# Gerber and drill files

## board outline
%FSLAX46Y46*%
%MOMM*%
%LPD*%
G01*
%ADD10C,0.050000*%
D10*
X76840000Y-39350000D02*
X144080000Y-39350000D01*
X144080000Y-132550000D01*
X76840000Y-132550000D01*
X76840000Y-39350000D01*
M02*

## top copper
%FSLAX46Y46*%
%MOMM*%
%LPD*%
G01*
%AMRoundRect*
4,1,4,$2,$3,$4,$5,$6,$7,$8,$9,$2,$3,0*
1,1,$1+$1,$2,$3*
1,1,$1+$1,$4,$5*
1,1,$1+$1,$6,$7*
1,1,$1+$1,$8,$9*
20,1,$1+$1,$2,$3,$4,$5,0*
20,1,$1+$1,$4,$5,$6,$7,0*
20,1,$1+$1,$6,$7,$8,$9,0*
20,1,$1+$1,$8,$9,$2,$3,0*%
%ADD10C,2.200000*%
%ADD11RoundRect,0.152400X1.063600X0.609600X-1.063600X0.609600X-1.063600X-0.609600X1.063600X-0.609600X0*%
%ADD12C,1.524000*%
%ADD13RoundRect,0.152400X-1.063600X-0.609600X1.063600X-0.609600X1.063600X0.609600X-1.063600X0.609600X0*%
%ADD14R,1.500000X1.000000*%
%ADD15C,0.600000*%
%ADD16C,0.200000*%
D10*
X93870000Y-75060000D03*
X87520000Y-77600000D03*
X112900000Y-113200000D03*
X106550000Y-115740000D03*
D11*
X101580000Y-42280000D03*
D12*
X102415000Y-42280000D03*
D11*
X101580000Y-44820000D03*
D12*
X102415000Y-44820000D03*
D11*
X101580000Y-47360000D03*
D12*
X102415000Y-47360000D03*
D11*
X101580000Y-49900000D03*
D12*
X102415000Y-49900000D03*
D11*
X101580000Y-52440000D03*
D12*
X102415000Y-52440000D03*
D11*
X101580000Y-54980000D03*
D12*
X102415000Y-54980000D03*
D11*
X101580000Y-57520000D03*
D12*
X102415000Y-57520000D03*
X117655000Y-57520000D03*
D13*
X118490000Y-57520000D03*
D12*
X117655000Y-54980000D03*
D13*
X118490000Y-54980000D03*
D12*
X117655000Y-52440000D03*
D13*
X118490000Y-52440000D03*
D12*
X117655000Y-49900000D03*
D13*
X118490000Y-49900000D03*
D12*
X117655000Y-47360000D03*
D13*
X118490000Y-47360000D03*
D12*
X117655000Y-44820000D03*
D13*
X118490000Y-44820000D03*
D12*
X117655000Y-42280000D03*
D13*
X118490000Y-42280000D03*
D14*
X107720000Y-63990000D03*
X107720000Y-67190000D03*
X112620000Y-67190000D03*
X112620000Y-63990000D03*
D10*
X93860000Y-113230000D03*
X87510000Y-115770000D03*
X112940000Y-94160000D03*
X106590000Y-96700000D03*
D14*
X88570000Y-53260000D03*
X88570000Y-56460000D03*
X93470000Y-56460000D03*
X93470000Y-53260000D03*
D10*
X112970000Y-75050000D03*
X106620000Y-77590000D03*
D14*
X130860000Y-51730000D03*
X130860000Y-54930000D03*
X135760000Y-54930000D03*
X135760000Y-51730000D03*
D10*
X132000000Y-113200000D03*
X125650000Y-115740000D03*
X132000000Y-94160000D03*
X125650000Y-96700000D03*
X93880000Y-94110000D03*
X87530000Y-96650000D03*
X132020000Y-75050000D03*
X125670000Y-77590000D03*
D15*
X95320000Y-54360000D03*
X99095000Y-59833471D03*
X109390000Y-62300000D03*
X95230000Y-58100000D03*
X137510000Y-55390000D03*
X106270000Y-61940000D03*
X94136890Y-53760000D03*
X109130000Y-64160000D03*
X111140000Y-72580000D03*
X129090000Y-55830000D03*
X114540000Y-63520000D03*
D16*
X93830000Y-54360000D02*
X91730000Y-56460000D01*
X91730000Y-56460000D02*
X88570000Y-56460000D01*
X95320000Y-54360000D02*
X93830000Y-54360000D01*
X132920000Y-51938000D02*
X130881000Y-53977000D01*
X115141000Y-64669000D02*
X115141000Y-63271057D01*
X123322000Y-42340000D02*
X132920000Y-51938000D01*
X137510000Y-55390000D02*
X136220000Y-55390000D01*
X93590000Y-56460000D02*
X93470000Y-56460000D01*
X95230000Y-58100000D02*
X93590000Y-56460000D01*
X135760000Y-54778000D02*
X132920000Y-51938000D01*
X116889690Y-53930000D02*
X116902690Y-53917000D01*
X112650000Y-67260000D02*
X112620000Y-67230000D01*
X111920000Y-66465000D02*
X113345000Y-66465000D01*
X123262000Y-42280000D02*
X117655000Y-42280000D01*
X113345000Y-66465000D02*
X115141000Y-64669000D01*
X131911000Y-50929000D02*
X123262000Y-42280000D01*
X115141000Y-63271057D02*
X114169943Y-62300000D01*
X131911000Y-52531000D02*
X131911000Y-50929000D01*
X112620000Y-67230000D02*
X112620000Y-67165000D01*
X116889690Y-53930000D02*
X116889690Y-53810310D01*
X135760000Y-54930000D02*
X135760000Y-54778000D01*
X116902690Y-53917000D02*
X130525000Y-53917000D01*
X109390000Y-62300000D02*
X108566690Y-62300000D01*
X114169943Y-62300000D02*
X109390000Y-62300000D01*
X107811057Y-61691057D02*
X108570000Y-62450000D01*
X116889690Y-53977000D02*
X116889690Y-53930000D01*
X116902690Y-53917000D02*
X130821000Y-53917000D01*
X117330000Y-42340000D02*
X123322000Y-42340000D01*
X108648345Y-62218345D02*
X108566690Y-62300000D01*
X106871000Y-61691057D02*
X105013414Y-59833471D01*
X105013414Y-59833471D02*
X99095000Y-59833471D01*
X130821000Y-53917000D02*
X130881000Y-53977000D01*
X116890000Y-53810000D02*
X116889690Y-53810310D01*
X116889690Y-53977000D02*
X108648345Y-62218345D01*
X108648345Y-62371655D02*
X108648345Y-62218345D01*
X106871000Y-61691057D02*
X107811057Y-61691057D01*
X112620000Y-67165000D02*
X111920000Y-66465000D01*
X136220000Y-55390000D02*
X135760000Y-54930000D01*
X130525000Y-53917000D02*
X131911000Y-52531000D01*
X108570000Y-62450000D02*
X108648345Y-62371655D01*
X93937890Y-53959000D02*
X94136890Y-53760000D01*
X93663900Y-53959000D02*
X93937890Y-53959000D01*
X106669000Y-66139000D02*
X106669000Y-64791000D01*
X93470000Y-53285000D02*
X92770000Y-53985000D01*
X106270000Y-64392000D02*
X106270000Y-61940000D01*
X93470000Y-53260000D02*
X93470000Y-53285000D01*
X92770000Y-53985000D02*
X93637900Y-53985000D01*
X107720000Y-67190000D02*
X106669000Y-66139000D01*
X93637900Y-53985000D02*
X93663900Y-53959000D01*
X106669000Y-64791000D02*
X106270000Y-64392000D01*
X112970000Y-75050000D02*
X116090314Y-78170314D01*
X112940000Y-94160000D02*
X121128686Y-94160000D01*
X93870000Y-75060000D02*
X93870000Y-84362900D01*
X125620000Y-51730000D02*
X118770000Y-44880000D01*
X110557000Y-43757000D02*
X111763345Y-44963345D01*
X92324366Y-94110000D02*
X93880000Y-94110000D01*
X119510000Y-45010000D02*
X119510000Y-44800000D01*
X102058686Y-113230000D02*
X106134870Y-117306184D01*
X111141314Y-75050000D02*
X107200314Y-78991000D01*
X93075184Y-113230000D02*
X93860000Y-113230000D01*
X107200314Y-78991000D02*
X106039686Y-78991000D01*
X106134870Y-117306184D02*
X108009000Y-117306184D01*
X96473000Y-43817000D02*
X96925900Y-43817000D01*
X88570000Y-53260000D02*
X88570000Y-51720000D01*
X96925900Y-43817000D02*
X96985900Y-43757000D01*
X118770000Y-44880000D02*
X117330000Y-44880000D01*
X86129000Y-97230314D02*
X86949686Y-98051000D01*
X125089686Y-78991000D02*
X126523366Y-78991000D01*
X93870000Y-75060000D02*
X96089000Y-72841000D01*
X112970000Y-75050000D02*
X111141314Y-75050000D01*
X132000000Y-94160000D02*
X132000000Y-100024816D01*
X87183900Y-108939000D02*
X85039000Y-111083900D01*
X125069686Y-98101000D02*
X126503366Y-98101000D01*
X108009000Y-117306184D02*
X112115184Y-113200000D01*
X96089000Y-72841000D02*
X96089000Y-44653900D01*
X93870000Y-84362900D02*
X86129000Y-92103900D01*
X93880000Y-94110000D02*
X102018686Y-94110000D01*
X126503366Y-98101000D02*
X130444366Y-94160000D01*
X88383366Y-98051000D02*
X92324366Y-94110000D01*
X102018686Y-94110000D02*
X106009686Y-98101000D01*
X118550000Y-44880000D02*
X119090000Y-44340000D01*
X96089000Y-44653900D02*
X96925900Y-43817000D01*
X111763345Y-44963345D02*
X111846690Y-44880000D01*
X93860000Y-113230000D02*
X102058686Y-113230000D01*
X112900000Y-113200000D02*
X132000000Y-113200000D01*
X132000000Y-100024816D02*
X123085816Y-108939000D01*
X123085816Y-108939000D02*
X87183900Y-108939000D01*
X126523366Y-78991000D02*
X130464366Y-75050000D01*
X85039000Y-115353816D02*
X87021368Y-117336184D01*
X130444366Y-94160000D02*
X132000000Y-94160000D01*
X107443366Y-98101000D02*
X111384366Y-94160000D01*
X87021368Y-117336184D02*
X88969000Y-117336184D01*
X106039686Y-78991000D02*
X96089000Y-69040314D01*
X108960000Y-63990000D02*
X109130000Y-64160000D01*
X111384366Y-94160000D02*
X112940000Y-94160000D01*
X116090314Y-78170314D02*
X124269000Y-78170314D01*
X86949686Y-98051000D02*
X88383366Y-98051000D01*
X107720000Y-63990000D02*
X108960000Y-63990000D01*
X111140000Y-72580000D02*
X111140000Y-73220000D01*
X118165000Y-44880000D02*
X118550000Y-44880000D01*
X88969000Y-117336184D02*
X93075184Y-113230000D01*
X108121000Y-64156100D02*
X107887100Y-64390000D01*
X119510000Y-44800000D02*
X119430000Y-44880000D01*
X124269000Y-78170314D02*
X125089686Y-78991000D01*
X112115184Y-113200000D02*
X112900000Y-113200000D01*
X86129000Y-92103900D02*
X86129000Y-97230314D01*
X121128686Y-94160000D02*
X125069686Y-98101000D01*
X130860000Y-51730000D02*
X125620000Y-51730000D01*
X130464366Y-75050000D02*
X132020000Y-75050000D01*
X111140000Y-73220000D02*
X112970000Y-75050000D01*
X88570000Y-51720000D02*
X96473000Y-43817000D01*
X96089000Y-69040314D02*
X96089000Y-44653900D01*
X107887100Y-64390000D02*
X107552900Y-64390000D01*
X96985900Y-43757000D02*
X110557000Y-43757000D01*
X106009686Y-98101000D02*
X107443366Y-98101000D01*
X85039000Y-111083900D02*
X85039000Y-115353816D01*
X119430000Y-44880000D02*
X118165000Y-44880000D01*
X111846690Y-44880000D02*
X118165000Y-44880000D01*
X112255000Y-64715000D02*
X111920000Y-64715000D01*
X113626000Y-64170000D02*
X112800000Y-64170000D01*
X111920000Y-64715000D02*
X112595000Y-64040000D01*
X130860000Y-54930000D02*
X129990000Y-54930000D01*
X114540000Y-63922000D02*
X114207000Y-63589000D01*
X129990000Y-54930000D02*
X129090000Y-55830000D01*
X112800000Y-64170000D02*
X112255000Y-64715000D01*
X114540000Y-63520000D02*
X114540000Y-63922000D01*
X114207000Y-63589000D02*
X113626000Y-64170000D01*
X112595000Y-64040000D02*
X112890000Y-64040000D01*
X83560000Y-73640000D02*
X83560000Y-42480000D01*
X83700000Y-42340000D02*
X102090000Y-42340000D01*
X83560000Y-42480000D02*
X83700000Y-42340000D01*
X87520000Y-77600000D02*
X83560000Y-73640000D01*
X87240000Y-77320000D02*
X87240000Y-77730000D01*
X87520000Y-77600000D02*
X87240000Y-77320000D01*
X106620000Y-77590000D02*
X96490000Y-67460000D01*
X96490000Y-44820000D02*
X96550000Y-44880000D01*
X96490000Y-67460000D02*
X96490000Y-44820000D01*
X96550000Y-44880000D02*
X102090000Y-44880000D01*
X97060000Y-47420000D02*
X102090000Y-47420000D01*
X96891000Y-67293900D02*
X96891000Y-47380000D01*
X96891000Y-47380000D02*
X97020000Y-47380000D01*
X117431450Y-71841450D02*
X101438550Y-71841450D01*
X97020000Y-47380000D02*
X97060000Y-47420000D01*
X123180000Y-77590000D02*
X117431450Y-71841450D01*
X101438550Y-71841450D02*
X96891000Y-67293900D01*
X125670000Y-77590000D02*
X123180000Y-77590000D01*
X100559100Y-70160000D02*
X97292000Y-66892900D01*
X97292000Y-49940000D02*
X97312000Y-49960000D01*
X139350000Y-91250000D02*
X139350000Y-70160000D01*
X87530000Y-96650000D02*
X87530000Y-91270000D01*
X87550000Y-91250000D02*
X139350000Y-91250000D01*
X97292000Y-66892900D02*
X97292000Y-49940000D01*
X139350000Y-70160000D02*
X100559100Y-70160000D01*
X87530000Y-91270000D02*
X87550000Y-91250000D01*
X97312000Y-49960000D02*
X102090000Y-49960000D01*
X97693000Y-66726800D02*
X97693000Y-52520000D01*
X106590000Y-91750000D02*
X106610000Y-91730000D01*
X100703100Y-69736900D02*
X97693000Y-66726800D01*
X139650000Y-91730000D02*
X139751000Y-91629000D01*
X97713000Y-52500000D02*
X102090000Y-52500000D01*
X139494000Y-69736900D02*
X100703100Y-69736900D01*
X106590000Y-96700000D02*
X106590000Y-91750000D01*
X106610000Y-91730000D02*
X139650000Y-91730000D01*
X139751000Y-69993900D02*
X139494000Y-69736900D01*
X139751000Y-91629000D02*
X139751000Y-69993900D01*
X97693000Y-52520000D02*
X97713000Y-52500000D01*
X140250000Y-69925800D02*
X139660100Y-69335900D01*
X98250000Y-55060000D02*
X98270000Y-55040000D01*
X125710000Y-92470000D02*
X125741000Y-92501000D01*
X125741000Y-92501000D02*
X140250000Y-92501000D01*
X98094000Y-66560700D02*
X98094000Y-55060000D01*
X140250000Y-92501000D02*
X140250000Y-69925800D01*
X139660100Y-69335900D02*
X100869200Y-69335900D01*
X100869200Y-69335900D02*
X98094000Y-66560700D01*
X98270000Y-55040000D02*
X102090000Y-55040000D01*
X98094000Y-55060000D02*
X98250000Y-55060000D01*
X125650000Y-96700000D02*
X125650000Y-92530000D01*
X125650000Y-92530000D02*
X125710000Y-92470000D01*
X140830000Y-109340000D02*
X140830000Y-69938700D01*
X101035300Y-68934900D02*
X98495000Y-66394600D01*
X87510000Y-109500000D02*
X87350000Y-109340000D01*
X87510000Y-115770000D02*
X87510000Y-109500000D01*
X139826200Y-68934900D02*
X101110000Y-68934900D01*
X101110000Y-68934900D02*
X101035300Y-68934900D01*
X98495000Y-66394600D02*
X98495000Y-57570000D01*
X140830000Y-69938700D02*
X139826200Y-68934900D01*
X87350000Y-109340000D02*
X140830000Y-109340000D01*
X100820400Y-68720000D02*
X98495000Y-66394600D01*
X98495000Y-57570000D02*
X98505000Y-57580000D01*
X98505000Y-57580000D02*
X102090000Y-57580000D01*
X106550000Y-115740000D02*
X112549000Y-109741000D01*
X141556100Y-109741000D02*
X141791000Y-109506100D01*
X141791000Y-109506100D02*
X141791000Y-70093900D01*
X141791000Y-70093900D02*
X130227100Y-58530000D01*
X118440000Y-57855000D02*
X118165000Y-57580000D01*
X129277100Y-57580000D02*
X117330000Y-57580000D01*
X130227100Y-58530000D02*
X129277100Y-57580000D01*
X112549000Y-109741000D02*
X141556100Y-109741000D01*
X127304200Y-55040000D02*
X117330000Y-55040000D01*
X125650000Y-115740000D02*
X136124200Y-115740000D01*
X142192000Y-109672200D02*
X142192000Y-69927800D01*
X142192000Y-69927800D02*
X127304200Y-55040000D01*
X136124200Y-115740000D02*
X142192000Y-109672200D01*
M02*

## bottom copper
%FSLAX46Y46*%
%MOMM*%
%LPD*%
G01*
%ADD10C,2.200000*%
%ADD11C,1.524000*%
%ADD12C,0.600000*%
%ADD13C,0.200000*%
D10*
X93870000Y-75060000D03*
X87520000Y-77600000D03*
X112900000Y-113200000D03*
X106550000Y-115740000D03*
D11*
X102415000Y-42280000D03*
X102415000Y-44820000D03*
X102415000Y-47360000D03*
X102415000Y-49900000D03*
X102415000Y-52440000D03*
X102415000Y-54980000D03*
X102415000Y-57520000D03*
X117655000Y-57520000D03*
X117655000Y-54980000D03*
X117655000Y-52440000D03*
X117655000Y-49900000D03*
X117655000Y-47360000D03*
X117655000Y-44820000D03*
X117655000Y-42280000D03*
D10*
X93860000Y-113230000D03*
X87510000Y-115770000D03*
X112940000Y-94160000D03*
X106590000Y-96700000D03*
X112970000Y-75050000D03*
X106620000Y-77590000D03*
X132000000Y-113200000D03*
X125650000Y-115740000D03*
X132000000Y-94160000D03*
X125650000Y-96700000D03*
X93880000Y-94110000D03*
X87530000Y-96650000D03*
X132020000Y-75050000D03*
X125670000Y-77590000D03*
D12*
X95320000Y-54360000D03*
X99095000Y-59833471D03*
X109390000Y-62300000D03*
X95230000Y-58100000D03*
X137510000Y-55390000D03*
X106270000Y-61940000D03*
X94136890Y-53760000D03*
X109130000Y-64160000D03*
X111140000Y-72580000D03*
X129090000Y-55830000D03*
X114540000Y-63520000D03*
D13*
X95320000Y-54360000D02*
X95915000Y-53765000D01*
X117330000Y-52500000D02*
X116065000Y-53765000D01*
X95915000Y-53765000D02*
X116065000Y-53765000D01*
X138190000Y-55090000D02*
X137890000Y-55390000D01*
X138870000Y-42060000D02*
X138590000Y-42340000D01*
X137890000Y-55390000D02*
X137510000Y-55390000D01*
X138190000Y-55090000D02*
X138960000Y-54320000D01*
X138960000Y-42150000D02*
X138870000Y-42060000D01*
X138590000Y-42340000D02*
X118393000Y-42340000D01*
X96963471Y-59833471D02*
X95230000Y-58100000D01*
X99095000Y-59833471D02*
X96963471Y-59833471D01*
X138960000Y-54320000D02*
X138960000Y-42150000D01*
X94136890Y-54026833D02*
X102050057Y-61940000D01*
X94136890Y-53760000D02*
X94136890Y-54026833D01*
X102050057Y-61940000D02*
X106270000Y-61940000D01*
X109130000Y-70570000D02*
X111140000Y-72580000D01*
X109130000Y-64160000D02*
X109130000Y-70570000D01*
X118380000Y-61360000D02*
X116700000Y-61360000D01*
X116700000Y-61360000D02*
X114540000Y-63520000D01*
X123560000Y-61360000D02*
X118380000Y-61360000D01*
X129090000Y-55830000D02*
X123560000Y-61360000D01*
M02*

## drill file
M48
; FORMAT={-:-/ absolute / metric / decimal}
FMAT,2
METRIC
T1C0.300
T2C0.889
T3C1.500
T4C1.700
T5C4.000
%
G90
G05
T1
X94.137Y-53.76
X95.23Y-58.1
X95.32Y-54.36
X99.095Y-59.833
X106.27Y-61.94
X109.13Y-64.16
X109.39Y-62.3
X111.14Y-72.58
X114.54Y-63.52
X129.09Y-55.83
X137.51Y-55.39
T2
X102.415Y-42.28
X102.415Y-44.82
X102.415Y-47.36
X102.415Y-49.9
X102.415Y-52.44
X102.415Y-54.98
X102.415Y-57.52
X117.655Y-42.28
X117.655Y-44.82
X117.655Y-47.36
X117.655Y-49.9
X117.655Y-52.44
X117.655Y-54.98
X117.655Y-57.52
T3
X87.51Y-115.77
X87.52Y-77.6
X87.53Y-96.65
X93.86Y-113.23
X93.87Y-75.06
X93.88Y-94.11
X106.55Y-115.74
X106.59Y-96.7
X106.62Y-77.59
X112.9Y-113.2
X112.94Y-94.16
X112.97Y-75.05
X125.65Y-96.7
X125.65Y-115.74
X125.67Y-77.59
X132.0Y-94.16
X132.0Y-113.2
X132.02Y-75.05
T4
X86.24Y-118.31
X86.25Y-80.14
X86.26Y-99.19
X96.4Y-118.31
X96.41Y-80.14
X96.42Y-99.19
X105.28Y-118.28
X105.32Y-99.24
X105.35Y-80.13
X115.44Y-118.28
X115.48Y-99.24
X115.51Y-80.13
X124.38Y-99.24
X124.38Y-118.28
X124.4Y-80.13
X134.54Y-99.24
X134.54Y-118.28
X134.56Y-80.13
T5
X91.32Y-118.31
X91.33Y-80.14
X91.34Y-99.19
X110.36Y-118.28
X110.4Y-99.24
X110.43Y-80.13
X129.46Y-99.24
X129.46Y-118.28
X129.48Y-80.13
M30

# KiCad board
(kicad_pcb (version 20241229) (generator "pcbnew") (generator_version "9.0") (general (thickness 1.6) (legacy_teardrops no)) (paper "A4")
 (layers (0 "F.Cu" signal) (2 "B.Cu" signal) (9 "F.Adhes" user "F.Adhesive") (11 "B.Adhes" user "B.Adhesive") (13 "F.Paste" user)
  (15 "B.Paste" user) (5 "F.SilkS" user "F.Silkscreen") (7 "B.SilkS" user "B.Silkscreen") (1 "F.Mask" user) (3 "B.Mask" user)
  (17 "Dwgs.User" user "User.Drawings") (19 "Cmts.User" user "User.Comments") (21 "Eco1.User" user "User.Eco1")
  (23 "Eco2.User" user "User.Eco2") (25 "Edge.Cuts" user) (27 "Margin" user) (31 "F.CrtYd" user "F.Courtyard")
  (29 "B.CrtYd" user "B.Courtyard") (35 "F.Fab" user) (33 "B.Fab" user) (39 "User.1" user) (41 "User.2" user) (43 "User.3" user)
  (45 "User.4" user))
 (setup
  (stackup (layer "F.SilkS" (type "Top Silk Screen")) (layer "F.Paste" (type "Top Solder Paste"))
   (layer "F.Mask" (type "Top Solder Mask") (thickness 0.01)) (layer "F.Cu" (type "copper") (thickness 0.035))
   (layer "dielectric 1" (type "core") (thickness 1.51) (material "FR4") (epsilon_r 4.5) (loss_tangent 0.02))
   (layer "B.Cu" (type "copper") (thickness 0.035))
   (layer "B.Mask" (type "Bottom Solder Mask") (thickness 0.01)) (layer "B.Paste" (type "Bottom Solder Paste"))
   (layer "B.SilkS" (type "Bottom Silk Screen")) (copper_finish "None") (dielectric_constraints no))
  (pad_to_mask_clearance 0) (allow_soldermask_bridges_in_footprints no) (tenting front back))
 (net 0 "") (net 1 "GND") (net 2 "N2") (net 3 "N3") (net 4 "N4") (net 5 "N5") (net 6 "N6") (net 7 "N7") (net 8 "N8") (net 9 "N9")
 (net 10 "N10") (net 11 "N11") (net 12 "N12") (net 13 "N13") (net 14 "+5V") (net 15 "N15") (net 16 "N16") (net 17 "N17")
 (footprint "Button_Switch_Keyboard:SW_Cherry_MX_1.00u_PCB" (layer "F.Cu") (at 93.87 75.06)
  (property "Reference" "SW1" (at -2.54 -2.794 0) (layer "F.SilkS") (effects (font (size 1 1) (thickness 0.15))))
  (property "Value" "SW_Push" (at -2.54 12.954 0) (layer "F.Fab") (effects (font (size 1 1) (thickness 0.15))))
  (pad "" np_thru_hole circle (at -7.62 5.08) (size 1.7 1.7) (drill 1.7) (layers "*.Cu" "*.Mask"))
  (pad "" np_thru_hole circle (at -2.54 5.08) (size 4 4) (drill 4) (layers "*.Cu" "*.Mask"))
  (pad "" np_thru_hole circle (at 2.54 5.08) (size 1.7 1.7) (drill 1.7) (layers "*.Cu" "*.Mask"))
  (pad "1" thru_hole circle (at 0 0) (size 2.2 2.2) (drill 1.5) (layers "*.Cu" "*.Mask") (remove_unused_layers no) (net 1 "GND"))
  (pad "2" thru_hole circle (at -6.35 2.54) (size 2.2 2.2) (drill 1.5) (layers "*.Cu" "*.Mask") (remove_unused_layers no) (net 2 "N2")))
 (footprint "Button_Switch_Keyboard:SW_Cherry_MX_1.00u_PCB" (layer "F.Cu") (at 112.9 113.2)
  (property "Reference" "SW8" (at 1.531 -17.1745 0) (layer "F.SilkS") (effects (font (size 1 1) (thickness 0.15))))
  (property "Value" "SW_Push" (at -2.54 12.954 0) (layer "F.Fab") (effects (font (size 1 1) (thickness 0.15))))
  (pad "" np_thru_hole circle (at -7.62 5.08) (size 1.7 1.7) (drill 1.7) (layers "*.Cu" "*.Mask"))
  (pad "" np_thru_hole circle (at -2.54 5.08) (size 4 4) (drill 4) (layers "*.Cu" "*.Mask"))
  (pad "" np_thru_hole circle (at 2.54 5.08) (size 1.7 1.7) (drill 1.7) (layers "*.Cu" "*.Mask"))
  (pad "1" thru_hole circle (at 0 0) (size 2.2 2.2) (drill 1.5) (layers "*.Cu" "*.Mask") (remove_unused_layers no) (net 1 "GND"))
  (pad "2" thru_hole circle (at -6.35 2.54) (size 2.2 2.2) (drill 1.5) (layers "*.Cu" "*.Mask") (remove_unused_layers no) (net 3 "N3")))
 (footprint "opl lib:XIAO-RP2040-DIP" (layer "F.Cu") (at 110.035 49.9)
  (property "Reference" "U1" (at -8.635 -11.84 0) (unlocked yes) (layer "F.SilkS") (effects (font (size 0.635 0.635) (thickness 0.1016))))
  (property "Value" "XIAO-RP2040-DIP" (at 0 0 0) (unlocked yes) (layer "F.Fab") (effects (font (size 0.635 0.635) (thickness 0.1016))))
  (pad "1" smd roundrect (at -8.455 -7.62 180) (size 2.432 1.524) (layers "F.Cu" "F.Mask") (roundrect_rratio 0.1) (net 2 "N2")
   (thermal_bridge_angle 45))
  (pad "1" thru_hole circle (at -7.62 -7.62 180) (size 1.524 1.524) (drill 0.889) (layers "*.Cu" "*.Mask") (remove_unused_layers no)
   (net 2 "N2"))
  (pad "2" smd roundrect (at -8.455 -5.08 180) (size 2.432 1.524) (layers "F.Cu" "F.Mask") (roundrect_rratio 0.1) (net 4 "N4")
   (thermal_bridge_angle 45))
  (pad "2" thru_hole circle (at -7.62 -5.08 180) (size 1.524 1.524) (drill 0.889) (layers "*.Cu" "*.Mask") (remove_unused_layers no)
   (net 4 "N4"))
  (pad "3" smd roundrect (at -8.455 -2.54 180) (size 2.432 1.524) (layers "F.Cu" "F.Mask") (roundrect_rratio 0.1) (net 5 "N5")
   (thermal_bridge_angle 45))
  (pad "3" thru_hole circle (at -7.62 -2.54 180) (size 1.524 1.524) (drill 0.889) (layers "*.Cu" "*.Mask") (remove_unused_layers no)
   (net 5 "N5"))
  (pad "4" smd roundrect (at -8.455 0 180) (size 2.432 1.524) (layers "F.Cu" "F.Mask") (roundrect_rratio 0.1) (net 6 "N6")
   (thermal_bridge_angle 45))
  (pad "4" thru_hole circle (at -7.62 0 180) (size 1.524 1.524) (drill 0.889) (layers "*.Cu" "*.Mask") (remove_unused_layers no)
   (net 6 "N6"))
  (pad "5" smd roundrect (at -8.455 2.54 180) (size 2.432 1.524) (layers "F.Cu" "F.Mask") (roundrect_rratio 0.1) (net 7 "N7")
   (thermal_bridge_angle 45))
  (pad "5" thru_hole circle (at -7.62 2.54 180) (size 1.524 1.524) (drill 0.889) (layers "*.Cu" "*.Mask") (remove_unused_layers no)
   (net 7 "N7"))
  (pad "6" smd roundrect (at -8.455 5.08 180) (size 2.432 1.524) (layers "F.Cu" "F.Mask") (roundrect_rratio 0.1) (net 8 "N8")
   (thermal_bridge_angle 45))
  (pad "6" thru_hole circle (at -7.62 5.08 180) (size 1.524 1.524) (drill 0.889) (layers "*.Cu" "*.Mask") (remove_unused_layers no)
   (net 8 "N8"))
  (pad "7" smd roundrect (at -8.455 7.62 180) (size 2.432 1.524) (layers "F.Cu" "F.Mask") (roundrect_rratio 0.1) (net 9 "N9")
   (thermal_bridge_angle 45))
  (pad "7" thru_hole circle (at -7.62 7.62 180) (size 1.524 1.524) (drill 0.889) (layers "*.Cu" "*.Mask") (remove_unused_layers no)
   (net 9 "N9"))
  (pad "8" thru_hole circle (at 7.62 7.62) (size 1.524 1.524) (drill 0.889) (layers "*.Cu" "*.Mask") (remove_unused_layers no) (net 3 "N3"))
  (pad "8" smd roundrect (at 8.455 7.62) (size 2.432 1.524) (layers "F.Cu" "F.Mask") (roundrect_rratio 0.1) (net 3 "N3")
   (thermal_bridge_angle 45))
  (pad "9" thru_hole circle (at 7.62 5.08) (size 1.524 1.524) (drill 0.889) (layers "*.Cu" "*.Mask") (remove_unused_layers no)
   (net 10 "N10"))
  (pad "9" smd roundrect (at 8.455 5.08) (size 2.432 1.524) (layers "F.Cu" "F.Mask") (roundrect_rratio 0.1) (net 10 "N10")
   (thermal_bridge_angle 45))
  (pad "10" thru_hole circle (at 7.62 2.54) (size 1.524 1.524) (drill 0.889) (layers "*.Cu" "*.Mask") (remove_unused_layers no)
   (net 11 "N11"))
  (pad "10" smd roundrect (at 8.455 2.54) (size 2.432 1.524) (layers "F.Cu" "F.Mask") (roundrect_rratio 0.1) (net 11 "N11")
   (thermal_bridge_angle 45))
  (pad "11" thru_hole circle (at 7.62 0) (size 1.524 1.524) (drill 0.889) (layers "*.Cu" "*.Mask") (remove_unused_layers no) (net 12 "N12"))
  (pad "11" smd roundrect (at 8.455 0) (size 2.432 1.524) (layers "F.Cu" "F.Mask") (roundrect_rratio 0.1) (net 12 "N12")
   (thermal_bridge_angle 45))
  (pad "12" thru_hole circle (at 7.62 -2.54) (size 1.524 1.524) (drill 0.889) (layers "*.Cu" "*.Mask") (remove_unused_layers no)
   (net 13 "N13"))
  (pad "12" smd roundrect (at 8.455 -2.54) (size 2.432 1.524) (layers "F.Cu" "F.Mask") (roundrect_rratio 0.1) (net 13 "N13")
   (thermal_bridge_angle 45))
  (pad "13" thru_hole circle (at 7.62 -5.08) (size 1.524 1.524) (drill 0.889) (layers "*.Cu" "*.Mask") (remove_unused_layers no)
   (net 1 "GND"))
  (pad "13" smd roundrect (at 8.455 -5.08) (size 2.432 1.524) (layers "F.Cu" "F.Mask") (roundrect_rratio 0.1) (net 1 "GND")
   (thermal_bridge_angle 45))
  (pad "14" thru_hole circle (at 7.62 -7.62) (size 1.524 1.524) (drill 0.889) (layers "*.Cu" "*.Mask") (remove_unused_layers no)
   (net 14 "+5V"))
  (pad "14" smd roundrect (at 8.455 -7.62) (size 2.432 1.524) (layers "F.Cu" "F.Mask") (roundrect_rratio 0.1) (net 14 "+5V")
   (thermal_bridge_angle 45)))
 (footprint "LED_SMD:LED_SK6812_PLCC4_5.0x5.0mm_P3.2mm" (layer "F.Cu") (at 110.17 65.59)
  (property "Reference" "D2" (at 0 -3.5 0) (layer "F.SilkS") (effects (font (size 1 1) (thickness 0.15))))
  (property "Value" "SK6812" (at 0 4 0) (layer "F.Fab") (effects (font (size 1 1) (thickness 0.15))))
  (pad "1" smd rect (at -2.45 -1.6 180) (size 1.5 1) (layers "F.Cu" "F.Mask" "F.Paste") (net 1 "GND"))
  (pad "2" smd rect (at -2.45 1.6 180) (size 1.5 1) (layers "F.Cu" "F.Mask" "F.Paste") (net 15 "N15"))
  (pad "3" smd rect (at 2.45 1.6 180) (size 1.5 1) (layers "F.Cu" "F.Mask" "F.Paste") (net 14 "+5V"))
  (pad "4" smd rect (at 2.45 -1.6 180) (size 1.5 1) (layers "F.Cu" "F.Mask" "F.Paste") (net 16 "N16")))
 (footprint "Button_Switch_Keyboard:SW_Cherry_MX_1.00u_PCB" (layer "F.Cu") (at 93.86 113.23)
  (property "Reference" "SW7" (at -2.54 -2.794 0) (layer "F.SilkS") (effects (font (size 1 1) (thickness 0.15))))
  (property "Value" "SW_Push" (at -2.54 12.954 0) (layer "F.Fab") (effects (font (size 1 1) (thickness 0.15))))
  (pad "" np_thru_hole circle (at -7.62 5.08) (size 1.7 1.7) (drill 1.7) (layers "*.Cu" "*.Mask"))
  (pad "" np_thru_hole circle (at -2.54 5.08) (size 4 4) (drill 4) (layers "*.Cu" "*.Mask"))
  (pad "" np_thru_hole circle (at 2.54 5.08) (size 1.7 1.7) (drill 1.7) (layers "*.Cu" "*.Mask"))
  (pad "1" thru_hole circle (at 0 0) (size 2.2 2.2) (drill 1.5) (layers "*.Cu" "*.Mask") (remove_unused_layers no) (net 1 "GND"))
  (pad "2" thru_hole circle (at -6.35 2.54) (size 2.2 2.2) (drill 1.5) (layers "*.Cu" "*.Mask") (remove_unused_layers no) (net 9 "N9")))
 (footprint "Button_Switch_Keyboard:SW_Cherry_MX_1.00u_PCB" (layer "F.Cu") (at 112.94 94.16)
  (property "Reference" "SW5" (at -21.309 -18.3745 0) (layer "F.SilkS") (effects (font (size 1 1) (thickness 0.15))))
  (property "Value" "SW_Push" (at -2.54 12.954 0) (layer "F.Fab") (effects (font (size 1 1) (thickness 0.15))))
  (pad "" np_thru_hole circle (at -7.62 5.08) (size 1.7 1.7) (drill 1.7) (layers "*.Cu" "*.Mask"))
  (pad "" np_thru_hole circle (at -2.54 5.08) (size 4 4) (drill 4) (layers "*.Cu" "*.Mask"))
  (pad "" np_thru_hole circle (at 2.54 5.08) (size 1.7 1.7) (drill 1.7) (layers "*.Cu" "*.Mask"))
  (pad "1" thru_hole circle (at 0 0) (size 2.2 2.2) (drill 1.5) (layers "*.Cu" "*.Mask") (remove_unused_layers no) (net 1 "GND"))
  (pad "2" thru_hole circle (at -6.35 2.54) (size 2.2 2.2) (drill 1.5) (layers "*.Cu" "*.Mask") (remove_unused_layers no) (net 7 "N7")))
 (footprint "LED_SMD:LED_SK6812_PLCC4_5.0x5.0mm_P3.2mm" (layer "F.Cu") (at 91.02 54.86)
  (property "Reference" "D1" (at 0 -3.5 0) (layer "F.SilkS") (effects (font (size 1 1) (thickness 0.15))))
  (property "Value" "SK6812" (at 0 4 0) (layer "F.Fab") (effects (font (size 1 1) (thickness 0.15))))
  (pad "1" smd rect (at -2.45 -1.6 180) (size 1.5 1) (layers "F.Cu" "F.Mask" "F.Paste") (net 1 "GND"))
  (pad "2" smd rect (at -2.45 1.6 180) (size 1.5 1) (layers "F.Cu" "F.Mask" "F.Paste") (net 11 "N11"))
  (pad "3" smd rect (at 2.45 1.6 180) (size 1.5 1) (layers "F.Cu" "F.Mask" "F.Paste") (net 14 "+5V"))
  (pad "4" smd rect (at 2.45 -1.6 180) (size 1.5 1) (layers "F.Cu" "F.Mask" "F.Paste") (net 15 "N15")))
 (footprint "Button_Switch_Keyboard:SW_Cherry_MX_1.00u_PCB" (layer "F.Cu") (at 112.97 75.05)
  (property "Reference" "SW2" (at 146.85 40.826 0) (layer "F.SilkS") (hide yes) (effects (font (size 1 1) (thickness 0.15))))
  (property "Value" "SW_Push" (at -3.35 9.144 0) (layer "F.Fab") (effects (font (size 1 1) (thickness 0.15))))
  (pad "" np_thru_hole circle (at -7.62 5.08) (size 1.7 1.7) (drill 1.7) (layers "*.Cu" "*.Mask"))
  (pad "" np_thru_hole circle (at -2.54 5.08) (size 4 4) (drill 4) (layers "*.Cu" "*.Mask"))
  (pad "" np_thru_hole circle (at 2.54 5.08) (size 1.7 1.7) (drill 1.7) (layers "*.Cu" "*.Mask"))
  (pad "1" thru_hole circle (at 0 0) (size 2.2 2.2) (drill 1.5) (layers "*.Cu" "*.Mask") (remove_unused_layers no) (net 1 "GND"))
  (pad "2" thru_hole circle (at -6.35 2.54) (size 2.2 2.2) (drill 1.5) (layers "*.Cu" "*.Mask") (remove_unused_layers no) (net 4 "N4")))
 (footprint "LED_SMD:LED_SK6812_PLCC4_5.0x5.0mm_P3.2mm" (layer "F.Cu") (at 133.31 53.33)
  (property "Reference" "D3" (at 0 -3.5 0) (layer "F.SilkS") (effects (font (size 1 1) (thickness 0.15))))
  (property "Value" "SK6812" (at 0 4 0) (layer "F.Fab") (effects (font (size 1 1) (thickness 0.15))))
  (pad "1" smd rect (at -2.45 -1.6 180) (size 1.5 1) (layers "F.Cu" "F.Mask" "F.Paste") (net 1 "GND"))
  (pad "2" smd rect (at -2.45 1.6 180) (size 1.5 1) (layers "F.Cu" "F.Mask" "F.Paste") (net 16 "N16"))
  (pad "3" smd rect (at 2.45 1.6 180) (size 1.5 1) (layers "F.Cu" "F.Mask" "F.Paste") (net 14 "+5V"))
  (pad "4" smd rect (at 2.45 -1.6 180) (size 1.5 1) (layers "F.Cu" "F.Mask" "F.Paste") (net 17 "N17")))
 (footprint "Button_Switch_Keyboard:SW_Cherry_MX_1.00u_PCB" (layer "F.Cu") (at 132 113.2)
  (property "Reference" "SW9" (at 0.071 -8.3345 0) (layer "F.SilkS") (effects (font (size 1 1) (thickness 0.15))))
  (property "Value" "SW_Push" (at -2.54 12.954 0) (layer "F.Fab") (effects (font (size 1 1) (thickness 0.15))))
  (pad "" np_thru_hole circle (at -7.62 5.08) (size 1.7 1.7) (drill 1.7) (layers "*.Cu" "*.Mask"))
  (pad "" np_thru_hole circle (at -2.54 5.08) (size 4 4) (drill 4) (layers "*.Cu" "*.Mask"))
  (pad "" np_thru_hole circle (at 2.54 5.08) (size 1.7 1.7) (drill 1.7) (layers "*.Cu" "*.Mask"))
  (pad "1" thru_hole circle (at 0 0) (size 2.2 2.2) (drill 1.5) (layers "*.Cu" "*.Mask") (remove_unused_layers no) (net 1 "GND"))
  (pad "2" thru_hole circle (at -6.35 2.54) (size 2.2 2.2) (drill 1.5) (layers "*.Cu" "*.Mask") (remove_unused_layers no) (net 10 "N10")))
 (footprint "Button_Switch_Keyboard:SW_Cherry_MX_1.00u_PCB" (layer "F.Cu") (at 132 94.16)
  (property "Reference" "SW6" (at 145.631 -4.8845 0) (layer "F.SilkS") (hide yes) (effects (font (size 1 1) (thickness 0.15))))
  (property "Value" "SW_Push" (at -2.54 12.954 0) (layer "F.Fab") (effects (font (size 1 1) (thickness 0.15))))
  (pad "" np_thru_hole circle (at -7.62 5.08) (size 1.7 1.7) (drill 1.7) (layers "*.Cu" "*.Mask"))
  (pad "" np_thru_hole circle (at -2.54 5.08) (size 4 4) (drill 4) (layers "*.Cu" "*.Mask"))
  (pad "" np_thru_hole circle (at 2.54 5.08) (size 1.7 1.7) (drill 1.7) (layers "*.Cu" "*.Mask"))
  (pad "1" thru_hole circle (at 0 0) (size 2.2 2.2) (drill 1.5) (layers "*.Cu" "*.Mask") (remove_unused_layers no) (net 1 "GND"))
  (pad "2" thru_hole circle (at -6.35 2.54) (size 2.2 2.2) (drill 1.5) (layers "*.Cu" "*.Mask") (remove_unused_layers no) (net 8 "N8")))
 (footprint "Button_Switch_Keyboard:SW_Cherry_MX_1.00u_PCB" (layer "F.Cu") (at 93.88 94.11)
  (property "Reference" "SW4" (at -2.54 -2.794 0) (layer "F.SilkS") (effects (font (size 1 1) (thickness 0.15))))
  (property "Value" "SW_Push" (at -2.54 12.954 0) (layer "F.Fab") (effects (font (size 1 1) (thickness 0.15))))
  (pad "" np_thru_hole circle (at -7.62 5.08) (size 1.7 1.7) (drill 1.7) (layers "*.Cu" "*.Mask"))
  (pad "" np_thru_hole circle (at -2.54 5.08) (size 4 4) (drill 4) (layers "*.Cu" "*.Mask"))
  (pad "" np_thru_hole circle (at 2.54 5.08) (size 1.7 1.7) (drill 1.7) (layers "*.Cu" "*.Mask"))
  (pad "1" thru_hole circle (at 0 0) (size 2.2 2.2) (drill 1.5) (layers "*.Cu" "*.Mask") (remove_unused_layers no) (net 1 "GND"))
  (pad "2" thru_hole circle (at -6.35 2.54) (size 2.2 2.2) (drill 1.5) (layers "*.Cu" "*.Mask") (remove_unused_layers no) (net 6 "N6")))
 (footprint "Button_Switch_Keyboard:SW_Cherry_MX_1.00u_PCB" (layer "F.Cu") (at 132.02 75.05)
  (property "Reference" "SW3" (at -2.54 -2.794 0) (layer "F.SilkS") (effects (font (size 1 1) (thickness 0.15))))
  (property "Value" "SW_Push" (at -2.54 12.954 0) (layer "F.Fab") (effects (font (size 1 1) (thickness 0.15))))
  (pad "" np_thru_hole circle (at -7.62 5.08) (size 1.7 1.7) (drill 1.7) (layers "*.Cu" "*.Mask"))
  (pad "" np_thru_hole circle (at -2.54 5.08) (size 4 4) (drill 4) (layers "*.Cu" "*.Mask"))
  (pad "" np_thru_hole circle (at 2.54 5.08) (size 1.7 1.7) (drill 1.7) (layers "*.Cu" "*.Mask"))
  (pad "1" thru_hole circle (at 0 0) (size 2.2 2.2) (drill 1.5) (layers "*.Cu" "*.Mask") (remove_unused_layers no) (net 1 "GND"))
  (pad "2" thru_hole circle (at -6.35 2.54) (size 2.2 2.2) (drill 1.5) (layers "*.Cu" "*.Mask") (remove_unused_layers no) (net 5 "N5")))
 (gr_rect (start 76.84 39.35) (end 144.08 132.55) (stroke (width 0.05) (type default)) (fill no) (layer "Edge.Cuts"))
 (segment (start 93.83 54.36) (end 91.73 56.46) (width 0.2) (layer "F.Cu") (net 11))
 (segment (start 91.73 56.46) (end 88.57 56.46) (width 0.2) (layer "F.Cu") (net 11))
 (segment (start 95.32 54.36) (end 93.83 54.36) (width 0.2) (layer "F.Cu") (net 11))
 (via (at 95.32 54.36) (size 0.6) (drill 0.3) (layers "F.Cu" "B.Cu") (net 11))
 (segment (start 95.32 54.36) (end 95.915 53.765) (width 0.2) (layer "B.Cu") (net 11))
 (segment (start 117.33 52.5) (end 116.065 53.765) (width 0.2) (layer "B.Cu") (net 11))
 (segment (start 95.915 53.765) (end 116.065 53.765) (width 0.2) (layer "B.Cu") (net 11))
 (segment (start 132.92 51.938) (end 130.881 53.977) (width 0.2) (layer "F.Cu") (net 14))
 (segment (start 115.141 64.669) (end 115.141 63.271057) (width 0.2) (layer "F.Cu") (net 14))
 (segment (start 123.322 42.34) (end 132.92 51.938) (width 0.2) (layer "F.Cu") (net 14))
 (segment (start 137.51 55.39) (end 136.22 55.39) (width 0.2) (layer "F.Cu") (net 14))
 (segment (start 93.59 56.46) (end 93.47 56.46) (width 0.2) (layer "F.Cu") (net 14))
 (segment (start 95.23 58.1) (end 93.59 56.46) (width 0.2) (layer "F.Cu") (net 14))
 (segment (start 135.76 54.778) (end 132.92 51.938) (width 0.2) (layer "F.Cu") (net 14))
 (segment (start 116.88969 53.93) (end 116.90269 53.917) (width 0.2) (layer "F.Cu") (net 14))
 (segment (start 112.65 67.26) (end 112.62 67.23) (width 0.2) (layer "F.Cu") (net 14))
 (segment (start 111.92 66.465) (end 113.345 66.465) (width 0.2) (layer "F.Cu") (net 14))
 (segment (start 123.262 42.28) (end 117.655 42.28) (width 0.2) (layer "F.Cu") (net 14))
 (segment (start 113.345 66.465) (end 115.141 64.669) (width 0.2) (layer "F.Cu") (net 14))
 (segment (start 131.911 50.929) (end 123.262 42.28) (width 0.2) (layer "F.Cu") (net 14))
 (segment (start 115.141 63.271057) (end 114.169943 62.3) (width 0.2) (layer "F.Cu") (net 14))
 (segment (start 131.911 52.531) (end 131.911 50.929) (width 0.2) (layer "F.Cu") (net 14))
 (segment (start 112.62 67.23) (end 112.62 67.165) (width 0.2) (layer "F.Cu") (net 14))
 (segment (start 116.88969 53.93) (end 116.88969 53.81031) (width 0.2) (layer "F.Cu") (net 14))
 (segment (start 135.76 54.93) (end 135.76 54.778) (width 0.2) (layer "F.Cu") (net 14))
 (segment (start 116.90269 53.917) (end 130.525 53.917) (width 0.2) (layer "F.Cu") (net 14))
 (segment (start 109.39 62.3) (end 108.56669 62.3) (width 0.2) (layer "F.Cu") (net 14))
 (segment (start 114.169943 62.3) (end 109.39 62.3) (width 0.2) (layer "F.Cu") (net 14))
 (segment (start 107.811057 61.691057) (end 108.57 62.45) (width 0.2) (layer "F.Cu") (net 14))
 (segment (start 116.88969 53.977) (end 116.88969 53.93) (width 0.2) (layer "F.Cu") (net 14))
 (segment (start 116.90269 53.917) (end 130.821 53.917) (width 0.2) (layer "F.Cu") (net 14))
 (segment (start 117.33 42.34) (end 123.322 42.34) (width 0.2) (layer "F.Cu") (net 14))
 (segment (start 108.648345 62.218345) (end 108.56669 62.3) (width 0.2) (layer "F.Cu") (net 14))
 (segment (start 106.871 61.691057) (end 105.013414 59.833471) (width 0.2) (layer "F.Cu") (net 14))
 (segment (start 105.013414 59.833471) (end 99.095 59.833471) (width 0.2) (layer "F.Cu") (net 14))
 (segment (start 130.821 53.917) (end 130.881 53.977) (width 0.2) (layer "F.Cu") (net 14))
 (segment (start 116.89 53.81) (end 116.88969 53.81031) (width 0.2) (layer "F.Cu") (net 14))
 (segment (start 116.88969 53.977) (end 108.648345 62.218345) (width 0.2) (layer "F.Cu") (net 14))
 (segment (start 108.648345 62.371655) (end 108.648345 62.218345) (width 0.2) (layer "F.Cu") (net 14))
 (segment (start 106.871 61.691057) (end 107.811057 61.691057) (width 0.2) (layer "F.Cu") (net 14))
 (segment (start 112.62 67.165) (end 111.92 66.465) (width 0.2) (layer "F.Cu") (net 14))
 (segment (start 136.22 55.39) (end 135.76 54.93) (width 0.2) (layer "F.Cu") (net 14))
 (segment (start 130.525 53.917) (end 131.911 52.531) (width 0.2) (layer "F.Cu") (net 14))
 (segment (start 108.57 62.45) (end 108.648345 62.371655) (width 0.2) (layer "F.Cu") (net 14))
 (via (at 99.095 59.833471) (size 0.6) (drill 0.3) (layers "F.Cu" "B.Cu") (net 14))
 (via (at 109.39 62.3) (size 0.6) (drill 0.3) (layers "F.Cu" "B.Cu") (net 14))
 (via (at 95.23 58.1) (size 0.6) (drill 0.3) (layers "F.Cu" "B.Cu") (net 14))
 (via (at 137.51 55.39) (size 0.6) (drill 0.3) (layers "F.Cu" "B.Cu") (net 14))
 (segment (start 138.19 55.09) (end 137.89 55.39) (width 0.2) (layer "B.Cu") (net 14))
 (segment (start 138.87 42.06) (end 138.59 42.34) (width 0.2) (layer "B.Cu") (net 14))
 (segment (start 137.89 55.39) (end 137.51 55.39) (width 0.2) (layer "B.Cu") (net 14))
 (segment (start 138.19 55.09) (end 138.96 54.32) (width 0.2) (layer "B.Cu") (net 14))
 (segment (start 138.96 42.15) (end 138.87 42.06) (width 0.2) (layer "B.Cu") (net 14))
 (segment (start 138.59 42.34) (end 118.393 42.34) (width 0.2) (layer "B.Cu") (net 14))
 (segment (start 96.963471 59.833471) (end 95.23 58.1) (width 0.2) (layer "B.Cu") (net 14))
 (segment (start 99.095 59.833471) (end 96.963471 59.833471) (width 0.2) (layer "B.Cu") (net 14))
 (segment (start 138.96 54.32) (end 138.96 42.15) (width 0.2) (layer "B.Cu") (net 14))
 (segment (start 93.93789 53.959) (end 94.13689 53.76) (width 0.2) (layer "F.Cu") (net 15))
 (segment (start 93.6639 53.959) (end 93.93789 53.959) (width 0.2) (layer "F.Cu") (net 15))
 (segment (start 106.669 66.139) (end 106.669 64.791) (width 0.2) (layer "F.Cu") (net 15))
 (segment (start 93.47 53.285) (end 92.77 53.985) (width 0.2) (layer "F.Cu") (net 15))
 (segment (start 106.27 64.392) (end 106.27 61.94) (width 0.2) (layer "F.Cu") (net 15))
 (segment (start 93.47 53.26) (end 93.47 53.285) (width 0.2) (layer "F.Cu") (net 15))
 (segment (start 92.77 53.985) (end 93.6379 53.985) (width 0.2) (layer "F.Cu") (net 15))
 (segment (start 107.72 67.19) (end 106.669 66.139) (width 0.2) (layer "F.Cu") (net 15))
 (segment (start 93.6379 53.985) (end 93.6639 53.959) (width 0.2) (layer "F.Cu") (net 15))
 (segment (start 106.669 64.791) (end 106.27 64.392) (width 0.2) (layer "F.Cu") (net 15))
 (via (at 106.27 61.94) (size 0.6) (drill 0.3) (layers "F.Cu" "B.Cu") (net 15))
 (via (at 94.13689 53.76) (size 0.6) (drill 0.3) (layers "F.Cu" "B.Cu") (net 15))
 (segment (start 94.13689 54.026833) (end 102.050057 61.94) (width 0.2) (layer "B.Cu") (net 15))
 (segment (start 94.13689 53.76) (end 94.13689 54.026833) (width 0.2) (layer "B.Cu") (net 15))
 (segment (start 102.050057 61.94) (end 106.27 61.94) (width 0.2) (layer "B.Cu") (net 15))
 (segment (start 112.97 75.05) (end 116.090314 78.170314) (width 0.2) (layer "F.Cu") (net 1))
 (segment (start 112.94 94.16) (end 121.128686 94.16) (width 0.2) (layer "F.Cu") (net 1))
 (segment (start 93.87 75.06) (end 93.87 84.3629) (width 0.2) (layer "F.Cu") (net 1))
 (segment (start 125.62 51.73) (end 118.77 44.88) (width 0.2) (layer "F.Cu") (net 1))
 (segment (start 110.557 43.757) (end 111.763345 44.963345) (width 0.2) (layer "F.Cu") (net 1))
 (segment (start 92.324366 94.11) (end 93.88 94.11) (width 0.2) (layer "F.Cu") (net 1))
 (segment (start 119.51 45.01) (end 119.51 44.8) (width 0.2) (layer "F.Cu") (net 1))
 (segment (start 102.058686 113.23) (end 106.13487 117.306184) (width 0.2) (layer "F.Cu") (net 1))
 (segment (start 111.141314 75.05) (end 107.200314 78.991) (width 0.2) (layer "F.Cu") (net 1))
 (segment (start 93.075184 113.23) (end 93.86 113.23) (width 0.2) (layer "F.Cu") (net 1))
 (segment (start 107.200314 78.991) (end 106.039686 78.991) (width 0.2) (layer "F.Cu") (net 1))
 (segment (start 106.13487 117.306184) (end 108.009 117.306184) (width 0.2) (layer "F.Cu") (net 1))
 (segment (start 96.473 43.817) (end 96.9259 43.817) (width 0.2) (layer "F.Cu") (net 1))
 (segment (start 88.57 53.26) (end 88.57 51.72) (width 0.2) (layer "F.Cu") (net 1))
 (segment (start 96.9259 43.817) (end 96.9859 43.757) (width 0.2) (layer "F.Cu") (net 1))
 (segment (start 118.77 44.88) (end 117.33 44.88) (width 0.2) (layer "F.Cu") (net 1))
 (segment (start 86.129 97.230314) (end 86.949686 98.051) (width 0.2) (layer "F.Cu") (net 1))
 (segment (start 125.089686 78.991) (end 126.523366 78.991) (width 0.2) (layer "F.Cu") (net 1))
 (segment (start 93.87 75.06) (end 96.089 72.841) (width 0.2) (layer "F.Cu") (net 1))
 (segment (start 112.97 75.05) (end 111.141314 75.05) (width 0.2) (layer "F.Cu") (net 1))
 (segment (start 132 94.16) (end 132 100.024816) (width 0.2) (layer "F.Cu") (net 1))
 (segment (start 87.1839 108.939) (end 85.039 111.0839) (width 0.2) (layer "F.Cu") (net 1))
 (segment (start 125.069686 98.101) (end 126.503366 98.101) (width 0.2) (layer "F.Cu") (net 1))
 (segment (start 108.009 117.306184) (end 112.115184 113.2) (width 0.2) (layer "F.Cu") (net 1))
 (segment (start 96.089 72.841) (end 96.089 44.6539) (width 0.2) (layer "F.Cu") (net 1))
 (segment (start 93.87 84.3629) (end 86.129 92.1039) (width 0.2) (layer "F.Cu") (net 1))
 (segment (start 93.88 94.11) (end 102.018686 94.11) (width 0.2) (layer "F.Cu") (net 1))
 (segment (start 126.503366 98.101) (end 130.444366 94.16) (width 0.2) (layer "F.Cu") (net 1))
 (segment (start 88.383366 98.051) (end 92.324366 94.11) (width 0.2) (layer "F.Cu") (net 1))
 (segment (start 102.018686 94.11) (end 106.009686 98.101) (width 0.2) (layer "F.Cu") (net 1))
 (segment (start 118.55 44.88) (end 119.09 44.34) (width 0.2) (layer "F.Cu") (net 1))
 (segment (start 96.089 44.6539) (end 96.9259 43.817) (width 0.2) (layer "F.Cu") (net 1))
 (segment (start 111.763345 44.963345) (end 111.84669 44.88) (width 0.2) (layer "F.Cu") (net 1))
 (segment (start 93.86 113.23) (end 102.058686 113.23) (width 0.2) (layer "F.Cu") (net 1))
 (segment (start 112.9 113.2) (end 132 113.2) (width 0.2) (layer "F.Cu") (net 1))
 (segment (start 132 100.024816) (end 123.085816 108.939) (width 0.2) (layer "F.Cu") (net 1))
 (segment (start 123.085816 108.939) (end 87.1839 108.939) (width 0.2) (layer "F.Cu") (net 1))
 (segment (start 126.523366 78.991) (end 130.464366 75.05) (width 0.2) (layer "F.Cu") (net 1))
 (segment (start 85.039 115.353816) (end 87.021368 117.336184) (width 0.2) (layer "F.Cu") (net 1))
 (segment (start 130.444366 94.16) (end 132 94.16) (width 0.2) (layer "F.Cu") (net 1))
 (segment (start 107.443366 98.101) (end 111.384366 94.16) (width 0.2) (layer "F.Cu") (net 1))
 (segment (start 87.021368 117.336184) (end 88.969 117.336184) (width 0.2) (layer "F.Cu") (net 1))
 (segment (start 106.039686 78.991) (end 96.089 69.040314) (width 0.2) (layer "F.Cu") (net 1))
 (segment (start 108.96 63.99) (end 109.13 64.16) (width 0.2) (layer "F.Cu") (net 1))
 (segment (start 111.384366 94.16) (end 112.94 94.16) (width 0.2) (layer "F.Cu") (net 1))
 (segment (start 116.090314 78.170314) (end 124.269 78.170314) (width 0.2) (layer "F.Cu") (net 1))
 (segment (start 86.949686 98.051) (end 88.383366 98.051) (width 0.2) (layer "F.Cu") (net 1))
 (segment (start 107.72 63.99) (end 108.96 63.99) (width 0.2) (layer "F.Cu") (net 1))
 (segment (start 111.14 72.58) (end 111.14 73.22) (width 0.2) (layer "F.Cu") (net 1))
 (segment (start 118.165 44.88) (end 118.55 44.88) (width 0.2) (layer "F.Cu") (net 1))
 (segment (start 88.969 117.336184) (end 93.075184 113.23) (width 0.2) (layer "F.Cu") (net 1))
 (segment (start 108.121 64.1561) (end 107.8871 64.39) (width 0.2) (layer "F.Cu") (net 1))
 (segment (start 119.51 44.8) (end 119.43 44.88) (width 0.2) (layer "F.Cu") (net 1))
 (segment (start 124.269 78.170314) (end 125.089686 78.991) (width 0.2) (layer "F.Cu") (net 1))
 (segment (start 112.115184 113.2) (end 112.9 113.2) (width 0.2) (layer "F.Cu") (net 1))
 (segment (start 86.129 92.1039) (end 86.129 97.230314) (width 0.2) (layer "F.Cu") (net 1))
 (segment (start 121.128686 94.16) (end 125.069686 98.101) (width 0.2) (layer "F.Cu") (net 1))
 (segment (start 130.86 51.73) (end 125.62 51.73) (width 0.2) (layer "F.Cu") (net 1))
 (segment (start 130.464366 75.05) (end 132.02 75.05) (width 0.2) (layer "F.Cu") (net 1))
 (segment (start 111.14 73.22) (end 112.97 75.05) (width 0.2) (layer "F.Cu") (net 1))
 (segment (start 88.57 51.72) (end 96.473 43.817) (width 0.2) (layer "F.Cu") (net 1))
 (segment (start 96.089 69.040314) (end 96.089 44.6539) (width 0.2) (layer "F.Cu") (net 1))
 (segment (start 107.8871 64.39) (end 107.5529 64.39) (width 0.2) (layer "F.Cu") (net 1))
 (segment (start 96.9859 43.757) (end 110.557 43.757) (width 0.2) (layer "F.Cu") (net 1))
 (segment (start 106.009686 98.101) (end 107.443366 98.101) (width 0.2) (layer "F.Cu") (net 1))
 (segment (start 85.039 111.0839) (end 85.039 115.353816) (width 0.2) (layer "F.Cu") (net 1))
 (segment (start 119.43 44.88) (end 118.165 44.88) (width 0.2) (layer "F.Cu") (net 1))
 (segment (start 111.84669 44.88) (end 118.165 44.88) (width 0.2) (layer "F.Cu") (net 1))
 (via (at 109.13 64.16) (size 0.6) (drill 0.3) (layers "F.Cu" "B.Cu") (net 1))
 (via (at 111.14 72.58) (size 0.6) (drill 0.3) (layers "F.Cu" "B.Cu") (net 1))
 (segment (start 109.13 70.57) (end 111.14 72.58) (width 0.2) (layer "B.Cu") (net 1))
 (segment (start 109.13 64.16) (end 109.13 70.57) (width 0.2) (layer "B.Cu") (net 1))
 (segment (start 112.255 64.715) (end 111.92 64.715) (width 0.2) (layer "F.Cu") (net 16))
 (segment (start 113.626 64.17) (end 112.8 64.17) (width 0.2) (layer "F.Cu") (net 16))
 (segment (start 111.92 64.715) (end 112.595 64.04) (width 0.2) (layer "F.Cu") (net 16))
 (segment (start 130.86 54.93) (end 129.99 54.93) (width 0.2) (layer "F.Cu") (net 16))
 (segment (start 114.54 63.922) (end 114.207 63.589) (width 0.2) (layer "F.Cu") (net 16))
 (segment (start 129.99 54.93) (end 129.09 55.83) (width 0.2) (layer "F.Cu") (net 16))
 (segment (start 112.8 64.17) (end 112.255 64.715) (width 0.2) (layer "F.Cu") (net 16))
 (segment (start 114.54 63.52) (end 114.54 63.922) (width 0.2) (layer "F.Cu") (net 16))
 (segment (start 114.207 63.589) (end 113.626 64.17) (width 0.2) (layer "F.Cu") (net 16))
 (segment (start 112.595 64.04) (end 112.89 64.04) (width 0.2) (layer "F.Cu") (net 16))
 (via (at 129.09 55.83) (size 0.6) (drill 0.3) (layers "F.Cu" "B.Cu") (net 16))
 (via (at 114.54 63.52) (size 0.6) (drill 0.3) (layers "F.Cu" "B.Cu") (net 16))
 (segment (start 118.38 61.36) (end 116.7 61.36) (width 0.2) (layer "B.Cu") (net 16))
 (segment (start 116.7 61.36) (end 114.54 63.52) (width 0.2) (layer "B.Cu") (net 16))
 (segment (start 123.56 61.36) (end 118.38 61.36) (width 0.2) (layer "B.Cu") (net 16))
 (segment (start 129.09 55.83) (end 123.56 61.36) (width 0.2) (layer "B.Cu") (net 16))
 (segment (start 83.56 73.64) (end 83.56 42.48) (width 0.2) (layer "F.Cu") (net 2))
 (segment (start 83.7 42.34) (end 102.09 42.34) (width 0.2) (layer "F.Cu") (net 2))
 (segment (start 83.56 42.48) (end 83.7 42.34) (width 0.2) (layer "F.Cu") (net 2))
 (segment (start 87.52 77.6) (end 83.56 73.64) (width 0.2) (layer "F.Cu") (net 2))
 (segment (start 87.24 77.32) (end 87.24 77.73) (width 0.2) (layer "F.Cu") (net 2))
 (segment (start 87.52 77.6) (end 87.24 77.32) (width 0.2) (layer "F.Cu") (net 2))
 (segment (start 106.62 77.59) (end 96.49 67.46) (width 0.2) (layer "F.Cu") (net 4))
 (segment (start 96.49 44.82) (end 96.55 44.88) (width 0.2) (layer "F.Cu") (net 4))
 (segment (start 96.49 67.46) (end 96.49 44.82) (width 0.2) (layer "F.Cu") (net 4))
 (segment (start 96.55 44.88) (end 102.09 44.88) (width 0.2) (layer "F.Cu") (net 4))
 (segment (start 97.06 47.42) (end 102.09 47.42) (width 0.2) (layer "F.Cu") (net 5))
 (segment (start 96.891 67.2939) (end 96.891 47.38) (width 0.2) (layer "F.Cu") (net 5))
 (segment (start 96.891 47.38) (end 97.02 47.38) (width 0.2) (layer "F.Cu") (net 5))
 (segment (start 117.43145 71.84145) (end 101.43855 71.84145) (width 0.2) (layer "F.Cu") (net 5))
 (segment (start 97.02 47.38) (end 97.06 47.42) (width 0.2) (layer "F.Cu") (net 5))
 (segment (start 123.18 77.59) (end 117.43145 71.84145) (width 0.2) (layer "F.Cu") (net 5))
 (segment (start 101.43855 71.84145) (end 96.891 67.2939) (width 0.2) (layer "F.Cu") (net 5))
 (segment (start 125.67 77.59) (end 123.18 77.59) (width 0.2) (layer "F.Cu") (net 5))
 (segment (start 100.5591 70.16) (end 97.292 66.8929) (width 0.2) (layer "F.Cu") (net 6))
 (segment (start 97.292 49.94) (end 97.312 49.96) (width 0.2) (layer "F.Cu") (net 6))
 (segment (start 139.35 91.25) (end 139.35 70.16) (width 0.2) (layer "F.Cu") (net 6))
 (segment (start 87.53 96.65) (end 87.53 91.27) (width 0.2) (layer "F.Cu") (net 6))
 (segment (start 87.55 91.25) (end 139.35 91.25) (width 0.2) (layer "F.Cu") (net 6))
 (segment (start 97.292 66.8929) (end 97.292 49.94) (width 0.2) (layer "F.Cu") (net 6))
 (segment (start 139.35 70.16) (end 100.5591 70.16) (width 0.2) (layer "F.Cu") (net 6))
 (segment (start 87.53 91.27) (end 87.55 91.25) (width 0.2) (layer "F.Cu") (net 6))
 (segment (start 97.312 49.96) (end 102.09 49.96) (width 0.2) (layer "F.Cu") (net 6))
 (segment (start 97.693 66.7268) (end 97.693 52.52) (width 0.2) (layer "F.Cu") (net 7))
 (segment (start 106.59 91.75) (end 106.61 91.73) (width 0.2) (layer "F.Cu") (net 7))
 (segment (start 100.7031 69.7369) (end 97.693 66.7268) (width 0.2) (layer "F.Cu") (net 7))
 (segment (start 139.65 91.73) (end 139.751 91.629) (width 0.2) (layer "F.Cu") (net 7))
 (segment (start 97.713 52.5) (end 102.09 52.5) (width 0.2) (layer "F.Cu") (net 7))
 (segment (start 139.494 69.7369) (end 100.7031 69.7369) (width 0.2) (layer "F.Cu") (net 7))
 (segment (start 106.59 96.7) (end 106.59 91.75) (width 0.2) (layer "F.Cu") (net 7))
 (segment (start 106.61 91.73) (end 139.65 91.73) (width 0.2) (layer "F.Cu") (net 7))
 (segment (start 139.751 69.9939) (end 139.494 69.7369) (width 0.2) (layer "F.Cu") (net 7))
 (segment (start 139.751 91.629) (end 139.751 69.9939) (width 0.2) (layer "F.Cu") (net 7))
 (segment (start 97.693 52.52) (end 97.713 52.5) (width 0.2) (layer "F.Cu") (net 7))
 (segment (start 140.25 69.9258) (end 139.6601 69.3359) (width 0.2) (layer "F.Cu") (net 8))
 (segment (start 98.25 55.06) (end 98.27 55.04) (width 0.2) (layer "F.Cu") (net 8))
 (segment (start 125.71 92.47) (end 125.741 92.501) (width 0.2) (layer "F.Cu") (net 8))
 (segment (start 125.741 92.501) (end 140.25 92.501) (width 0.2) (layer "F.Cu") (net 8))
 (segment (start 98.094 66.5607) (end 98.094 55.06) (width 0.2) (layer "F.Cu") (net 8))
 (segment (start 140.25 92.501) (end 140.25 69.9258) (width 0.2) (layer "F.Cu") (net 8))
 (segment (start 139.6601 69.3359) (end 100.8692 69.3359) (width 0.2) (layer "F.Cu") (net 8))
 (segment (start 100.8692 69.3359) (end 98.094 66.5607) (width 0.2) (layer "F.Cu") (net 8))
 (segment (start 98.27 55.04) (end 102.09 55.04) (width 0.2) (layer "F.Cu") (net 8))
 (segment (start 98.094 55.06) (end 98.25 55.06) (width 0.2) (layer "F.Cu") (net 8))
 (segment (start 125.65 96.7) (end 125.65 92.53) (width 0.2) (layer "F.Cu") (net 8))
 (segment (start 125.65 92.53) (end 125.71 92.47) (width 0.2) (layer "F.Cu") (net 8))
 (segment (start 140.83 109.34) (end 140.83 69.9387) (width 0.2) (layer "F.Cu") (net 9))
 (segment (start 101.0353 68.9349) (end 98.495 66.3946) (width 0.2) (layer "F.Cu") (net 9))
 (segment (start 87.51 109.5) (end 87.35 109.34) (width 0.2) (layer "F.Cu") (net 9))
 (segment (start 87.51 115.77) (end 87.51 109.5) (width 0.2) (layer "F.Cu") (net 9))
 (segment (start 139.8262 68.9349) (end 101.11 68.9349) (width 0.2) (layer "F.Cu") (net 9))
 (segment (start 101.11 68.9349) (end 101.0353 68.9349) (width 0.2) (layer "F.Cu") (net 9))
 (segment (start 98.495 66.3946) (end 98.495 57.57) (width 0.2) (layer "F.Cu") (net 9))
 (segment (start 140.83 69.9387) (end 139.8262 68.9349) (width 0.2) (layer "F.Cu") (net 9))
 (segment (start 87.35 109.34) (end 140.83 109.34) (width 0.2) (layer "F.Cu") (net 9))
 (segment (start 100.8204 68.72) (end 98.495 66.3946) (width 0.2) (layer "F.Cu") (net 9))
 (segment (start 98.495 57.57) (end 98.505 57.58) (width 0.2) (layer "F.Cu") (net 9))
 (segment (start 98.505 57.58) (end 102.09 57.58) (width 0.2) (layer "F.Cu") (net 9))
 (segment (start 106.55 115.74) (end 112.549 109.741) (width 0.2) (layer "F.Cu") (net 3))
 (segment (start 141.5561 109.741) (end 141.791 109.5061) (width 0.2) (layer "F.Cu") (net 3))
 (segment (start 141.791 109.5061) (end 141.791 70.0939) (width 0.2) (layer "F.Cu") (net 3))
 (segment (start 141.791 70.0939) (end 130.2271 58.53) (width 0.2) (layer "F.Cu") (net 3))
 (segment (start 118.44 57.855) (end 118.165 57.58) (width 0.2) (layer "F.Cu") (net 3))
 (segment (start 129.2771 57.58) (end 117.33 57.58) (width 0.2) (layer "F.Cu") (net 3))
 (segment (start 130.2271 58.53) (end 129.2771 57.58) (width 0.2) (layer "F.Cu") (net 3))
 (segment (start 112.549 109.741) (end 141.5561 109.741) (width 0.2) (layer "F.Cu") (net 3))
 (segment (start 127.3042 55.04) (end 117.33 55.04) (width 0.2) (layer "F.Cu") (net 10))
 (segment (start 125.65 115.74) (end 136.1242 115.74) (width 0.2) (layer "F.Cu") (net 10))
 (segment (start 142.192 109.6722) (end 142.192 69.9278) (width 0.2) (layer "F.Cu") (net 10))
 (segment (start 142.192 69.9278) (end 127.3042 55.04) (width 0.2) (layer "F.Cu") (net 10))
 (segment (start 136.1242 115.74) (end 142.192 109.6722) (width 0.2) (layer "F.Cu") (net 10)))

